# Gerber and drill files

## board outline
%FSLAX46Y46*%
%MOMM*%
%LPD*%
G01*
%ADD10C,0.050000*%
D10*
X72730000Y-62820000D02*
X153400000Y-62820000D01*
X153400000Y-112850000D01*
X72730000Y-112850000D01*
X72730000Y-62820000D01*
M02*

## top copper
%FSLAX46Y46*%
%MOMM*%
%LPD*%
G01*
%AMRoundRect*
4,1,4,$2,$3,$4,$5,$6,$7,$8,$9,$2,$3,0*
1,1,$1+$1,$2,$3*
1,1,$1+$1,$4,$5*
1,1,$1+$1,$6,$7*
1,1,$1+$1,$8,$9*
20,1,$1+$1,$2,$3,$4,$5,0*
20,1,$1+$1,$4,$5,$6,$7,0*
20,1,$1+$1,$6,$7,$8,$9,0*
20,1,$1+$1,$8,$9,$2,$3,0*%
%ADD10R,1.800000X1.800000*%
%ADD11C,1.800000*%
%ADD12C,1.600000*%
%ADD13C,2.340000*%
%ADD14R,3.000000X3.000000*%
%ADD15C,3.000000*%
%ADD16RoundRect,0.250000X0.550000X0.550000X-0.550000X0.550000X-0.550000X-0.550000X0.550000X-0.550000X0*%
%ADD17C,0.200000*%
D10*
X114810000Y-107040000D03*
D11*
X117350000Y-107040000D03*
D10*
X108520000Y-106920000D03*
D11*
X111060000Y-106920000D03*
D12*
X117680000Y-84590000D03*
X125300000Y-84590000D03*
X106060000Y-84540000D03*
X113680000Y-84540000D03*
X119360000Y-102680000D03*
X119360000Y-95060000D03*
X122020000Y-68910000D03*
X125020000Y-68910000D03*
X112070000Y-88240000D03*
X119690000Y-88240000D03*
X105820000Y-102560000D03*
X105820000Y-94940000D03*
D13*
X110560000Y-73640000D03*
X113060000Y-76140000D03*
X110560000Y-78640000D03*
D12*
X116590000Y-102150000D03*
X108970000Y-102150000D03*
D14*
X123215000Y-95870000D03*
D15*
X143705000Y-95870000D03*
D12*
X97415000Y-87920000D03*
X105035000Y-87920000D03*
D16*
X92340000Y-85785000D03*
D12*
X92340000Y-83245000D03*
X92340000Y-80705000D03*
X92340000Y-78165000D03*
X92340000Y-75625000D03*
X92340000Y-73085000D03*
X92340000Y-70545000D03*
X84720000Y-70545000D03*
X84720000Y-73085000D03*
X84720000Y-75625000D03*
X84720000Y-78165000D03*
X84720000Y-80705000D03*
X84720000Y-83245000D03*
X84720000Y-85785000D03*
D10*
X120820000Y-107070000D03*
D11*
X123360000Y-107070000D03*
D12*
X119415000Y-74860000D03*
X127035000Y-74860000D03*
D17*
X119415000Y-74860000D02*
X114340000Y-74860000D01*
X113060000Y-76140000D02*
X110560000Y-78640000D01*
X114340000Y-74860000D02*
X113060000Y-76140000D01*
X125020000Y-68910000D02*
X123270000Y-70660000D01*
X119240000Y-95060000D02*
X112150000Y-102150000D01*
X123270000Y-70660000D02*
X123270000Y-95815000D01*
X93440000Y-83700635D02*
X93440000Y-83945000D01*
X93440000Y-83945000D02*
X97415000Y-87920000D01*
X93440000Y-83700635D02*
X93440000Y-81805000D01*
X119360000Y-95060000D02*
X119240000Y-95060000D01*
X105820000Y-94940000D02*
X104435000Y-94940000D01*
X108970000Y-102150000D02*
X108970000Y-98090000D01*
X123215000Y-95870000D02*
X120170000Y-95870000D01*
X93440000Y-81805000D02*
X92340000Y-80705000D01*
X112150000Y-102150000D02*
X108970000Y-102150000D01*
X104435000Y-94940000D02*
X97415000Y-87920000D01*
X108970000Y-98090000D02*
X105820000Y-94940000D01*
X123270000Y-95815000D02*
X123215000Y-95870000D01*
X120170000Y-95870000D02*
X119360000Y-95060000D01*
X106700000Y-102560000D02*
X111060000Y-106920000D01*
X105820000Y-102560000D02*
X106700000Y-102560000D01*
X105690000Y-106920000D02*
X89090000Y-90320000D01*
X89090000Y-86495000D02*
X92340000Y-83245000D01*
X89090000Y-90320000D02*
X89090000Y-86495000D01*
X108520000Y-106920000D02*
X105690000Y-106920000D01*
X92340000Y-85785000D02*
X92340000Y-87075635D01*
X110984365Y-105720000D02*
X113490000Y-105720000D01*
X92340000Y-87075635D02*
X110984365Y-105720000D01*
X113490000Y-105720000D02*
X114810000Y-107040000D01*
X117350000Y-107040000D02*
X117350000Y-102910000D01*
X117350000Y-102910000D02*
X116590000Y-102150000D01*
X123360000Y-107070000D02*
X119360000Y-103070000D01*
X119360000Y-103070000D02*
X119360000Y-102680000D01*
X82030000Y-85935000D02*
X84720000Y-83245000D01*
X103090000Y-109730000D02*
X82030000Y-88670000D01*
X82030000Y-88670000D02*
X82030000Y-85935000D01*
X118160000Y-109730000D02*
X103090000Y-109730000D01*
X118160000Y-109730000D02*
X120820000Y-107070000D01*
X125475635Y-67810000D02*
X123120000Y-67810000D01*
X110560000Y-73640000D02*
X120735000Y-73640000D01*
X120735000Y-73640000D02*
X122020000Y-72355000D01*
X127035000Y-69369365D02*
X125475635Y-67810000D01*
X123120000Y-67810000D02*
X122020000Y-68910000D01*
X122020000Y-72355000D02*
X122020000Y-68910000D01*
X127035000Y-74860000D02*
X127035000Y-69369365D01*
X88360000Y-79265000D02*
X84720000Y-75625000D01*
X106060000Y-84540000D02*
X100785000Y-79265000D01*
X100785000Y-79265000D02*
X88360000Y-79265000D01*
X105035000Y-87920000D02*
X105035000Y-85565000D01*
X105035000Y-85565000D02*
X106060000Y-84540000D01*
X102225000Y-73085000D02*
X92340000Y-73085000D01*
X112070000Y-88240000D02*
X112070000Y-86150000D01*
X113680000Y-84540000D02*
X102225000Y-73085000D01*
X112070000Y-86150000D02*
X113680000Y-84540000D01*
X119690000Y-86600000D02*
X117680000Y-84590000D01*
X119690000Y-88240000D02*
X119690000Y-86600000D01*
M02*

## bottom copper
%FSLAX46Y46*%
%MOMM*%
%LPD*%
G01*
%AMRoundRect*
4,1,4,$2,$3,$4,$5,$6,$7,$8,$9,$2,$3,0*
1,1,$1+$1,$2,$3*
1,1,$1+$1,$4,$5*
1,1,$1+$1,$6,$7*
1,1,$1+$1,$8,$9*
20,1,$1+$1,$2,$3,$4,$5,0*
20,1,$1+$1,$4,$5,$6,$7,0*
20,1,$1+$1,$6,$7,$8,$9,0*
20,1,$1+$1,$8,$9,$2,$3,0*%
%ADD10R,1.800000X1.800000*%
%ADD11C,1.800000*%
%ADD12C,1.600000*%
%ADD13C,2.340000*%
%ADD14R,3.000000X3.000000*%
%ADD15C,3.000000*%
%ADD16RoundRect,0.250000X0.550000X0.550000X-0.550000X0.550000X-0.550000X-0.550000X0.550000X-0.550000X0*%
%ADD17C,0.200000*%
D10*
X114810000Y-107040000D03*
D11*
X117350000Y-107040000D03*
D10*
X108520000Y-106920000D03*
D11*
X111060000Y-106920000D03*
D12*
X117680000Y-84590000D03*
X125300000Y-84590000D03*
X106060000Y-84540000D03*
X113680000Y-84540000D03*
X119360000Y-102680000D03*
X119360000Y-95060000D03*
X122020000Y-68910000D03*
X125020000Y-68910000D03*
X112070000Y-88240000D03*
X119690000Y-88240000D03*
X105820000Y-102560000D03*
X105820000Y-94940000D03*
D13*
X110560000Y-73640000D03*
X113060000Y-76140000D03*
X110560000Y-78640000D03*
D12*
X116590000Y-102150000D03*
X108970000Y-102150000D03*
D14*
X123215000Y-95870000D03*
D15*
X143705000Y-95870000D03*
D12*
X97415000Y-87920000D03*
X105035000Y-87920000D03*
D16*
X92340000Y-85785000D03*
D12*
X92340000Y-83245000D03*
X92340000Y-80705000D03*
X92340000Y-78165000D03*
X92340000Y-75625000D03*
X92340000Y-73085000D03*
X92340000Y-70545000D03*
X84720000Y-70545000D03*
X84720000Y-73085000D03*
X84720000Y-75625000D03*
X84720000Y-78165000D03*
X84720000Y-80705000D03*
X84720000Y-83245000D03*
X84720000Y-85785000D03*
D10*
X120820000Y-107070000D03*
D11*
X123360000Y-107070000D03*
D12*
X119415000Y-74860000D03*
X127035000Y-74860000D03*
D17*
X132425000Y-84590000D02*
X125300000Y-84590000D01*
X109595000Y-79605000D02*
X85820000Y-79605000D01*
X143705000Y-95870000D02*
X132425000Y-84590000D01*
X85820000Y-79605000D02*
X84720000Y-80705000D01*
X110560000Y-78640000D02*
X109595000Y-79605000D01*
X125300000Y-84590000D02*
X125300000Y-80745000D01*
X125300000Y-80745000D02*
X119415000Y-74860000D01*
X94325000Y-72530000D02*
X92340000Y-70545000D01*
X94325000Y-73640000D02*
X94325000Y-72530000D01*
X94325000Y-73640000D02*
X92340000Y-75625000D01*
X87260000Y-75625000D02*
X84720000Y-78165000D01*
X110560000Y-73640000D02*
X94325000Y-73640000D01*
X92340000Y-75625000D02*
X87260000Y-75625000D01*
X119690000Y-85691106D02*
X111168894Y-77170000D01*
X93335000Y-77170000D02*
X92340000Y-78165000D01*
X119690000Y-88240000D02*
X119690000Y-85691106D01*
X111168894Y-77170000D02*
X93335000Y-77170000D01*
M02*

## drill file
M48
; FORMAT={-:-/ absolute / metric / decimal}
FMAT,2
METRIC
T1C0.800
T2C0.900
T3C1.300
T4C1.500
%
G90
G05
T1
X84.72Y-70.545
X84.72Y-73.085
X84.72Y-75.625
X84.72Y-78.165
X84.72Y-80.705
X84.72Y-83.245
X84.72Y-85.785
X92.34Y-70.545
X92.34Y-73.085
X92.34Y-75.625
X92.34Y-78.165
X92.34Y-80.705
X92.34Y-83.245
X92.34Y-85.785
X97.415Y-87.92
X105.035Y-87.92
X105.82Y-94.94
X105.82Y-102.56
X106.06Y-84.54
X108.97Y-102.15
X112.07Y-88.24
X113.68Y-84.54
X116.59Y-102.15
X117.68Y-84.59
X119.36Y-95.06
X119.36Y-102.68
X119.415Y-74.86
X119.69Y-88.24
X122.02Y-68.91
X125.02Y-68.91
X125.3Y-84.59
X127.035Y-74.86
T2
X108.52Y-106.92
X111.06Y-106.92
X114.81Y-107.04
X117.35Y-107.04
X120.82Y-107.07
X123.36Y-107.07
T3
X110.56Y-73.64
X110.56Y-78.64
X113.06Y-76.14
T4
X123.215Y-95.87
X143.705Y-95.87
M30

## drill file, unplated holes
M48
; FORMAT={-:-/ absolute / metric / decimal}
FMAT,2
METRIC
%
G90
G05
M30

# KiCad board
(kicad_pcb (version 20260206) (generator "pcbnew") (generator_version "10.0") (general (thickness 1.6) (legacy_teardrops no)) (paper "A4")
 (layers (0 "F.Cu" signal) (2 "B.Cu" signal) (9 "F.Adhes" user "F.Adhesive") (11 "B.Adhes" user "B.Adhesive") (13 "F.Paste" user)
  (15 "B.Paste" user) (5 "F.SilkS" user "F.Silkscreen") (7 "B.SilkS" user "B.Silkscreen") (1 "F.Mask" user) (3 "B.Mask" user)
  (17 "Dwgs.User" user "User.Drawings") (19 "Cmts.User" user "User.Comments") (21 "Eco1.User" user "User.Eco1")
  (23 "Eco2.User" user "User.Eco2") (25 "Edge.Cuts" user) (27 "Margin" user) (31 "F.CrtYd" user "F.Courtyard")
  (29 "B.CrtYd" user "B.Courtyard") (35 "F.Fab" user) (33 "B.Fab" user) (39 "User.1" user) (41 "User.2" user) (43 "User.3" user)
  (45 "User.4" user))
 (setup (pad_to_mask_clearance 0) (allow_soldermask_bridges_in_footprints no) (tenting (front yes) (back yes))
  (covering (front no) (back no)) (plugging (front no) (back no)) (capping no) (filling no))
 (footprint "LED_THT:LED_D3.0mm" (layer "F.Cu") (at 114.81 107.04)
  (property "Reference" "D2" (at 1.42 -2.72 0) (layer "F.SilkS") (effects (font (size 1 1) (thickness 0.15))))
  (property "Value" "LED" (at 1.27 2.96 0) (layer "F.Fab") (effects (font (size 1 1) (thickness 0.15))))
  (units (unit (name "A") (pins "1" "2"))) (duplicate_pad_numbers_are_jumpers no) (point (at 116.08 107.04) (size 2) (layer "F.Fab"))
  (pad "1" thru_hole rect (at 0 0) (size 1.8 1.8) (drill 0.9) (layers "*.Cu" "*.Mask") (remove_unused_layers no) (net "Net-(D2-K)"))
  (pad "2" thru_hole circle (at 2.54 0) (size 1.8 1.8) (drill 0.9) (layers "*.Cu" "*.Mask") (remove_unused_layers no) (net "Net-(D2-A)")))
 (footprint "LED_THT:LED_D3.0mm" (layer "F.Cu") (at 108.52 106.92)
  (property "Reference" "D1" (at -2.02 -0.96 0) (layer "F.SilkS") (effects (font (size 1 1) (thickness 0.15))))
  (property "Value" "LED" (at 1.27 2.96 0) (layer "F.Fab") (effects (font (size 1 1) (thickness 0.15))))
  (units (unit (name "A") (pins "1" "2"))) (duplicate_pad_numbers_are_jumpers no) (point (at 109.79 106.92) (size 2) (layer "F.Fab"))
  (pad "1" thru_hole rect (at 0 0) (size 1.8 1.8) (drill 0.9) (layers "*.Cu" "*.Mask") (remove_unused_layers no) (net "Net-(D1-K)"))
  (pad "2" thru_hole circle (at 2.54 0) (size 1.8 1.8) (drill 0.9) (layers "*.Cu" "*.Mask") (remove_unused_layers no) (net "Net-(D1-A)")))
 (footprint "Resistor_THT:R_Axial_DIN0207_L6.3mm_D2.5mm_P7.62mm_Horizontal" (layer "F.Cu") (at 117.68 84.59)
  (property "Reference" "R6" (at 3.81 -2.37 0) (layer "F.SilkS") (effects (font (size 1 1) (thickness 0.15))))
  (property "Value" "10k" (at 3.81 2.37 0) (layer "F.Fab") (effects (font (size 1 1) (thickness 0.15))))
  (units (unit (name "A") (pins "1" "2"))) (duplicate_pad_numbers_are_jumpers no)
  (pad "1" thru_hole circle (at 0 0) (size 1.6 1.6) (drill 0.8) (layers "*.Cu" "*.Mask") (remove_unused_layers no) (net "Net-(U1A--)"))
  (pad "2" thru_hole circle (at 7.62 0) (size 1.6 1.6) (drill 0.8) (layers "*.Cu" "*.Mask") (remove_unused_layers no) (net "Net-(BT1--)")))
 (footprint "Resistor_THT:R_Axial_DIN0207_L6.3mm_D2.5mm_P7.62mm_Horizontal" (layer "F.Cu") (at 106.06 84.54)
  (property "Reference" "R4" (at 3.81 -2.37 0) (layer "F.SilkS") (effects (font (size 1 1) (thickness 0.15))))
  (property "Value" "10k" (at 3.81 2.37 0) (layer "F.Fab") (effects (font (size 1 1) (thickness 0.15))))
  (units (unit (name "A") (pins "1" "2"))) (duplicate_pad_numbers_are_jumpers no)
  (pad "1" thru_hole circle (at 0 0) (size 1.6 1.6) (drill 0.8) (layers "*.Cu" "*.Mask") (remove_unused_layers no) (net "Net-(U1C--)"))
  (pad "2" thru_hole circle (at 7.62 0) (size 1.6 1.6) (drill 0.8) (layers "*.Cu" "*.Mask") (remove_unused_layers no) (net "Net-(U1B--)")))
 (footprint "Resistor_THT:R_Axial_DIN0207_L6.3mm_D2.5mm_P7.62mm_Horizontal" (layer "F.Cu") (at 119.36 102.68 90)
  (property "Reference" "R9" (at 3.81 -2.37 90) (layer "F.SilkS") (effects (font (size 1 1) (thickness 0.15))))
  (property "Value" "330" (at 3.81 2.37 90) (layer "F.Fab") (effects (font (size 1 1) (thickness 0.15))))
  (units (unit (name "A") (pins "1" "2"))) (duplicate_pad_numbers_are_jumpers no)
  (pad "1" thru_hole circle (at 0 0 90) (size 1.6 1.6) (drill 0.8) (layers "*.Cu" "*.Mask") (remove_unused_layers no) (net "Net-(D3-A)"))
  (pad "2" thru_hole circle (at 7.62 0 90) (size 1.6 1.6) (drill 0.8) (layers "*.Cu" "*.Mask") (remove_unused_layers no) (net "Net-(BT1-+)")))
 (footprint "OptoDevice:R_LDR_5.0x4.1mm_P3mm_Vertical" (layer "F.Cu") (at 122.02 68.91)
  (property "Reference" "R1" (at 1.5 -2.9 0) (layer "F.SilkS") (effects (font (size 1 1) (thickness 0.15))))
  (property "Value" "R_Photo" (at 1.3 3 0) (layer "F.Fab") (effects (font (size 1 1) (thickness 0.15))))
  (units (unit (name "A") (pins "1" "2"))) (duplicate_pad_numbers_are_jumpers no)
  (pad "1" thru_hole circle (at 0 0) (size 1.6 1.6) (drill 0.8) (layers "*.Cu" "*.Mask") (remove_unused_layers no) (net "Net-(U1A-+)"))
  (pad "2" thru_hole circle (at 3 0) (size 1.6 1.6) (drill 0.8) (layers "*.Cu" "*.Mask") (remove_unused_layers no) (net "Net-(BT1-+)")))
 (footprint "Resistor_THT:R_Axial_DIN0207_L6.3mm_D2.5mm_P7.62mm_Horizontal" (layer "F.Cu") (at 112.07 88.24)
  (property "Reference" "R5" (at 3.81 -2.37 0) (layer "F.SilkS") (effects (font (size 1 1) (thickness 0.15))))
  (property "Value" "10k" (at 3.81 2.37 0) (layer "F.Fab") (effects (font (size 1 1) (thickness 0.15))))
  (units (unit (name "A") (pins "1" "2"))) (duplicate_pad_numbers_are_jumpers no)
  (pad "1" thru_hole circle (at 0 0) (size 1.6 1.6) (drill 0.8) (layers "*.Cu" "*.Mask") (remove_unused_layers no) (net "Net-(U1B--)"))
  (pad "2" thru_hole circle (at 7.62 0) (size 1.6 1.6) (drill 0.8) (layers "*.Cu" "*.Mask") (remove_unused_layers no) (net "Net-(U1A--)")))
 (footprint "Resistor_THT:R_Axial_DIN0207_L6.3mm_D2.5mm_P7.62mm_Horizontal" (layer "F.Cu") (at 105.82 102.56 90)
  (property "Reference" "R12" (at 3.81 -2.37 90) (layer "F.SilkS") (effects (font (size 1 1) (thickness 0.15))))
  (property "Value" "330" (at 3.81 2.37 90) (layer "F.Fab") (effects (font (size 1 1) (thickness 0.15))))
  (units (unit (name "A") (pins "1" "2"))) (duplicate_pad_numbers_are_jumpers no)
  (pad "1" thru_hole circle (at 0 0 90) (size 1.6 1.6) (drill 0.8) (layers "*.Cu" "*.Mask") (remove_unused_layers no) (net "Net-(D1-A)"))
  (pad "2" thru_hole circle (at 7.62 0 90) (size 1.6 1.6) (drill 0.8) (layers "*.Cu" "*.Mask") (remove_unused_layers no) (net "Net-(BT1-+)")))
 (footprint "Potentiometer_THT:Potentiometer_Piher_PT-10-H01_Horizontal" (layer "F.Cu") (at 110.56 73.64)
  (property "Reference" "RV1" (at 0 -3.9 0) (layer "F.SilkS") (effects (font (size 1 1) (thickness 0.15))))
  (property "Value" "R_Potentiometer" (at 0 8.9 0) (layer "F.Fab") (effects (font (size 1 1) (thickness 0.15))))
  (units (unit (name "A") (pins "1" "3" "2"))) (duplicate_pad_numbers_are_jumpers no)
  (pad "1" thru_hole circle (at 0 0) (size 2.34 2.34) (drill 1.3) (layers "*.Cu" "*.Mask") (remove_unused_layers no) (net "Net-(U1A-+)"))
  (pad "2" thru_hole circle (at 2.5 2.5) (size 2.34 2.34) (drill 1.3) (layers "*.Cu" "*.Mask") (remove_unused_layers no) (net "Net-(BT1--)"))
  (pad "3" thru_hole circle (at 0 5) (size 2.34 2.34) (drill 1.3) (layers "*.Cu" "*.Mask") (remove_unused_layers no) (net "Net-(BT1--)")))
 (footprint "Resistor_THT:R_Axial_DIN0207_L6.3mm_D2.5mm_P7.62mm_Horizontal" (layer "F.Cu") (at 116.59 102.15 180)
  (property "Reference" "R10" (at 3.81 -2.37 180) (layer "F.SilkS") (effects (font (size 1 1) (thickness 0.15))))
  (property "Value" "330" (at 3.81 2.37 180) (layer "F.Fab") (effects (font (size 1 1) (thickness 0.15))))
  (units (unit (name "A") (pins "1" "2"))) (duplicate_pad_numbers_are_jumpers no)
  (pad "1" thru_hole circle (at 0 0 180) (size 1.6 1.6) (drill 0.8) (layers "*.Cu" "*.Mask") (remove_unused_layers no) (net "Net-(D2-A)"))
  (pad "2" thru_hole circle (at 7.62 0 180) (size 1.6 1.6) (drill 0.8) (layers "*.Cu" "*.Mask") (remove_unused_layers no)
   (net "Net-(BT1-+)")))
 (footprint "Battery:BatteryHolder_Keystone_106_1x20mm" (layer "F.Cu") (at 123.215 95.87)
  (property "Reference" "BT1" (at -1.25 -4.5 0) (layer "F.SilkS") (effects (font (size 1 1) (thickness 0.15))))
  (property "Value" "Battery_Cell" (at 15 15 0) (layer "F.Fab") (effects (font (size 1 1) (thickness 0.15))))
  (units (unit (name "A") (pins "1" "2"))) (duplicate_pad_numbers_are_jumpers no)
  (pad "1" thru_hole rect (at 0 0) (size 3 3) (drill 1.5) (layers "*.Cu" "*.Mask") (remove_unused_layers no) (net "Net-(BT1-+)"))
  (pad "2" thru_hole circle (at 20.49 0) (size 3 3) (drill 1.5) (layers "*.Cu" "*.Mask") (remove_unused_layers no) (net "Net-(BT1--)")))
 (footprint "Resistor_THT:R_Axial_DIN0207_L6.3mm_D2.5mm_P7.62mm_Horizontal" (layer "F.Cu") (at 97.415 87.92)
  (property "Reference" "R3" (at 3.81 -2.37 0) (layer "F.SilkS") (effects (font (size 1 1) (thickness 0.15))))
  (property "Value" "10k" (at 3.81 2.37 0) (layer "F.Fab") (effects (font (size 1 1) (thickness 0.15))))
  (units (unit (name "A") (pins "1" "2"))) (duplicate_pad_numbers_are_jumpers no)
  (pad "1" thru_hole circle (at 0 0) (size 1.6 1.6) (drill 0.8) (layers "*.Cu" "*.Mask") (remove_unused_layers no) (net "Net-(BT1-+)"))
  (pad "2" thru_hole circle (at 7.62 0) (size 1.6 1.6) (drill 0.8) (layers "*.Cu" "*.Mask") (remove_unused_layers no) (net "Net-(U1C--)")))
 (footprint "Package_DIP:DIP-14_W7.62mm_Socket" (layer "F.Cu") (at 92.34 85.785 180)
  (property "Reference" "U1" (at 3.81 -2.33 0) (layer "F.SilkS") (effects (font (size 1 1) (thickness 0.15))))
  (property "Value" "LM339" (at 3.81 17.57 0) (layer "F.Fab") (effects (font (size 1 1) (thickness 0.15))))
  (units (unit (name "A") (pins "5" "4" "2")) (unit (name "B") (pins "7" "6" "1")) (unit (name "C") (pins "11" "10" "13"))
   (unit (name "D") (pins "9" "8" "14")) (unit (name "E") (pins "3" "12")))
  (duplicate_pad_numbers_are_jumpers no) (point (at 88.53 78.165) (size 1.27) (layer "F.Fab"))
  (pad "1" thru_hole roundrect (at 0 0 180) (size 1.6 1.6) (drill 0.8) (layers "*.Cu" "*.Mask") (remove_unused_layers no)
   (roundrect_rratio 0.15625) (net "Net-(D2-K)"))
  (pad "2" thru_hole circle (at 0 2.54 180) (size 1.6 1.6) (drill 0.8) (layers "*.Cu" "*.Mask") (remove_unused_layers no) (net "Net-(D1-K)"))
  (pad "3" thru_hole circle (at 0 5.08 180) (size 1.6 1.6) (drill 0.8) (layers "*.Cu" "*.Mask") (remove_unused_layers no)
   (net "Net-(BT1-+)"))
  (pad "4" thru_hole circle (at 0 7.62 180) (size 1.6 1.6) (drill 0.8) (layers "*.Cu" "*.Mask") (remove_unused_layers no)
   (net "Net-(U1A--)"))
  (pad "5" thru_hole circle (at 0 10.16 180) (size 1.6 1.6) (drill 0.8) (layers "*.Cu" "*.Mask") (remove_unused_layers no)
   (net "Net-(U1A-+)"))
  (pad "6" thru_hole circle (at 0 12.7 180) (size 1.6 1.6) (drill 0.8) (layers "*.Cu" "*.Mask") (remove_unused_layers no)
   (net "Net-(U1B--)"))
  (pad "7" thru_hole circle (at 0 15.24 180) (size 1.6 1.6) (drill 0.8) (layers "*.Cu" "*.Mask") (remove_unused_layers no)
   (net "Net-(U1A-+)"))
  (pad "8" thru_hole circle (at 7.62 15.24 180) (size 1.6 1.6) (drill 0.8) (layers "*.Cu" "*.Mask") (remove_unused_layers no))
  (pad "9" thru_hole circle (at 7.62 12.7 180) (size 1.6 1.6) (drill 0.8) (layers "*.Cu" "*.Mask") (remove_unused_layers no))
  (pad "10" thru_hole circle (at 7.62 10.16 180) (size 1.6 1.6) (drill 0.8) (layers "*.Cu" "*.Mask") (remove_unused_layers no)
   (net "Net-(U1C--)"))
  (pad "11" thru_hole circle (at 7.62 7.62 180) (size 1.6 1.6) (drill 0.8) (layers "*.Cu" "*.Mask") (remove_unused_layers no)
   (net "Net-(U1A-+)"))
  (pad "12" thru_hole circle (at 7.62 5.08 180) (size 1.6 1.6) (drill 0.8) (layers "*.Cu" "*.Mask") (remove_unused_layers no)
   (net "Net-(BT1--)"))
  (pad "13" thru_hole circle (at 7.62 2.54 180) (size 1.6 1.6) (drill 0.8) (layers "*.Cu" "*.Mask") (remove_unused_layers no)
   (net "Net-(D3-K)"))
  (pad "14" thru_hole circle (at 7.62 0 180) (size 1.6 1.6) (drill 0.8) (layers "*.Cu" "*.Mask") (remove_unused_layers no)))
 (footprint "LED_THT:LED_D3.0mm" (layer "F.Cu") (at 120.82 107.07)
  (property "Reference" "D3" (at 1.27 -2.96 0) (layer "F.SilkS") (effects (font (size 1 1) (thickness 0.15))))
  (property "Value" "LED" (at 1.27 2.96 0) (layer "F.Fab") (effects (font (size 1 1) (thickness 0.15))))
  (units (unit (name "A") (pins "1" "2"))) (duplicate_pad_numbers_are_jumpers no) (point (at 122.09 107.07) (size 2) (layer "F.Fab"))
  (pad "1" thru_hole rect (at 0 0) (size 1.8 1.8) (drill 0.9) (layers "*.Cu" "*.Mask") (remove_unused_layers no) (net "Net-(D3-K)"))
  (pad "2" thru_hole circle (at 2.54 0) (size 1.8 1.8) (drill 0.9) (layers "*.Cu" "*.Mask") (remove_unused_layers no) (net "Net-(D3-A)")))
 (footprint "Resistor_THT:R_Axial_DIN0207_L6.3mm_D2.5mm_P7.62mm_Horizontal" (layer "F.Cu") (at 119.415 74.86)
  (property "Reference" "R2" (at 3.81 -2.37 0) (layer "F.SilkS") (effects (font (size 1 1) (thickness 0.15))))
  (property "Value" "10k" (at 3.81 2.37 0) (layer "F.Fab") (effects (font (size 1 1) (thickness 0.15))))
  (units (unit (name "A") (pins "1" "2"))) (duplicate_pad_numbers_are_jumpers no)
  (pad "1" thru_hole circle (at 0 0) (size 1.6 1.6) (drill 0.8) (layers "*.Cu" "*.Mask") (remove_unused_layers no) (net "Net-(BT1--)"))
  (pad "2" thru_hole circle (at 7.62 0) (size 1.6 1.6) (drill 0.8) (layers "*.Cu" "*.Mask") (remove_unused_layers no) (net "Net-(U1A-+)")))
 (gr_rect (start 72.73 62.82) (end 153.4 112.85) (stroke (width 0.05) (type default)) (fill no) (layer "Edge.Cuts"))
 (segment (start 119.415 74.86) (end 114.34 74.86) (width 0.2) (layer "F.Cu") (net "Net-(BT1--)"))
 (segment (start 113.06 76.14) (end 110.56 78.64) (width 0.2) (layer "F.Cu") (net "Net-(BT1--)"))
 (segment (start 114.34 74.86) (end 113.06 76.14) (width 0.2) (layer "F.Cu") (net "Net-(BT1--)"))
 (segment (start 132.425 84.59) (end 125.3 84.59) (width 0.2) (layer "B.Cu") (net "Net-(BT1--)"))
 (segment (start 109.595 79.605) (end 85.82 79.605) (width 0.2) (layer "B.Cu") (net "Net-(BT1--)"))
 (segment (start 143.705 95.87) (end 132.425 84.59) (width 0.2) (layer "B.Cu") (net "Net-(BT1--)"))
 (segment (start 85.82 79.605) (end 84.72 80.705) (width 0.2) (layer "B.Cu") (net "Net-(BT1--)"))
 (segment (start 110.56 78.64) (end 109.595 79.605) (width 0.2) (layer "B.Cu") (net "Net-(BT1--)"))
 (segment (start 125.3 84.59) (end 125.3 80.745) (width 0.2) (layer "B.Cu") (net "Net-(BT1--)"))
 (segment (start 125.3 80.745) (end 119.415 74.86) (width 0.2) (layer "B.Cu") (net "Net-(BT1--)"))
 (segment (start 125.02 68.91) (end 123.27 70.66) (width 0.2) (layer "F.Cu") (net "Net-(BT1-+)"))
 (segment (start 119.24 95.06) (end 112.15 102.15) (width 0.2) (layer "F.Cu") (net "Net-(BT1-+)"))
 (segment (start 123.27 70.66) (end 123.27 95.815) (width 0.2) (layer "F.Cu") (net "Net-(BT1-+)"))
 (segment (start 93.44 83.700635) (end 93.44 83.945) (width 0.2) (layer "F.Cu") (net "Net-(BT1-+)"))
 (segment (start 93.44 83.945) (end 97.415 87.92) (width 0.2) (layer "F.Cu") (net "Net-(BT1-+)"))
 (segment (start 93.44 83.700635) (end 93.44 81.805) (width 0.2) (layer "F.Cu") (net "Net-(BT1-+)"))
 (segment (start 119.36 95.06) (end 119.24 95.06) (width 0.2) (layer "F.Cu") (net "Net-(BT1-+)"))
 (segment (start 105.82 94.94) (end 104.435 94.94) (width 0.2) (layer "F.Cu") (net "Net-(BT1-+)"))
 (segment (start 108.97 102.15) (end 108.97 98.09) (width 0.2) (layer "F.Cu") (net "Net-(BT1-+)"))
 (segment (start 123.215 95.87) (end 120.17 95.87) (width 0.2) (layer "F.Cu") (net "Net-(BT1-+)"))
 (segment (start 93.44 81.805) (end 92.34 80.705) (width 0.2) (layer "F.Cu") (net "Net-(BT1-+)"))
 (segment (start 112.15 102.15) (end 108.97 102.15) (width 0.2) (layer "F.Cu") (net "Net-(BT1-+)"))
 (segment (start 104.435 94.94) (end 97.415 87.92) (width 0.2) (layer "F.Cu") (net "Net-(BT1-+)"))
 (segment (start 108.97 98.09) (end 105.82 94.94) (width 0.2) (layer "F.Cu") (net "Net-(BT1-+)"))
 (segment (start 123.27 95.815) (end 123.215 95.87) (width 0.2) (layer "F.Cu") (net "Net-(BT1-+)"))
 (segment (start 120.17 95.87) (end 119.36 95.06) (width 0.2) (layer "F.Cu") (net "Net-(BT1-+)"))
 (segment (start 106.7 102.56) (end 111.06 106.92) (width 0.2) (layer "F.Cu") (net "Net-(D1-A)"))
 (segment (start 105.82 102.56) (end 106.7 102.56) (width 0.2) (layer "F.Cu") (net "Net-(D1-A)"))
 (segment (start 105.69 106.92) (end 89.09 90.32) (width 0.2) (layer "F.Cu") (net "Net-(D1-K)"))
 (segment (start 89.09 86.495) (end 92.34 83.245) (width 0.2) (layer "F.Cu") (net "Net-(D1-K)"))
 (segment (start 89.09 90.32) (end 89.09 86.495) (width 0.2) (layer "F.Cu") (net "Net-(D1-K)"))
 (segment (start 108.52 106.92) (end 105.69 106.92) (width 0.2) (layer "F.Cu") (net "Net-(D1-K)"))
 (segment (start 92.34 85.785) (end 92.34 87.075635) (width 0.2) (layer "F.Cu") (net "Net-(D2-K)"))
 (segment (start 110.984365 105.72) (end 113.49 105.72) (width 0.2) (layer "F.Cu") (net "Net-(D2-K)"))
 (segment (start 92.34 87.075635) (end 110.984365 105.72) (width 0.2) (layer "F.Cu") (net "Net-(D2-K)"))
 (segment (start 113.49 105.72) (end 114.81 107.04) (width 0.2) (layer "F.Cu") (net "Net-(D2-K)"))
 (segment (start 117.35 107.04) (end 117.35 102.91) (width 0.2) (layer "F.Cu") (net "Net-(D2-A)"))
 (segment (start 117.35 102.91) (end 116.59 102.15) (width 0.2) (layer "F.Cu") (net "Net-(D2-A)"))
 (segment (start 123.36 107.07) (end 119.36 103.07) (width 0.2) (layer "F.Cu") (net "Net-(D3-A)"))
 (segment (start 119.36 103.07) (end 119.36 102.68) (width 0.2) (layer "F.Cu") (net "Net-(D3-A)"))
 (segment (start 82.03 85.935) (end 84.72 83.245) (width 0.2) (layer "F.Cu") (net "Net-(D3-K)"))
 (segment (start 103.09 109.73) (end 82.03 88.67) (width 0.2) (layer "F.Cu") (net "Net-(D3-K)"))
 (segment (start 82.03 88.67) (end 82.03 85.935) (width 0.2) (layer "F.Cu") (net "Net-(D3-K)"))
 (segment (start 118.16 109.73) (end 103.09 109.73) (width 0.2) (layer "F.Cu") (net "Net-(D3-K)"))
 (segment (start 118.16 109.73) (end 120.82 107.07) (width 0.2) (layer "F.Cu") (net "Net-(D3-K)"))
 (segment (start 125.475635 67.81) (end 123.12 67.81) (width 0.2) (layer "F.Cu") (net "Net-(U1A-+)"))
 (segment (start 110.56 73.64) (end 120.735 73.64) (width 0.2) (layer "F.Cu") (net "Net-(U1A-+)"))
 (segment (start 120.735 73.64) (end 122.02 72.355) (width 0.2) (layer "F.Cu") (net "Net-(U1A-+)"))
 (segment (start 127.035 69.369365) (end 125.475635 67.81) (width 0.2) (layer "F.Cu") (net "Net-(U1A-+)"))
 (segment (start 123.12 67.81) (end 122.02 68.91) (width 0.2) (layer "F.Cu") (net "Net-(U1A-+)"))
 (segment (start 122.02 72.355) (end 122.02 68.91) (width 0.2) (layer "F.Cu") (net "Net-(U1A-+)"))
 (segment (start 127.035 74.86) (end 127.035 69.369365) (width 0.2) (layer "F.Cu") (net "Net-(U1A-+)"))
 (segment (start 94.325 72.53) (end 92.34 70.545) (width 0.2) (layer "B.Cu") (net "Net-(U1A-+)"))
 (segment (start 94.325 73.64) (end 94.325 72.53) (width 0.2) (layer "B.Cu") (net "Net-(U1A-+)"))
 (segment (start 94.325 73.64) (end 92.34 75.625) (width 0.2) (layer "B.Cu") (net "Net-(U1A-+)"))
 (segment (start 87.26 75.625) (end 84.72 78.165) (width 0.2) (layer "B.Cu") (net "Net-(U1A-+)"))
 (segment (start 110.56 73.64) (end 94.325 73.64) (width 0.2) (layer "B.Cu") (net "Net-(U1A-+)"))
 (segment (start 92.34 75.625) (end 87.26 75.625) (width 0.2) (layer "B.Cu") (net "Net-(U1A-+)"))
 (segment (start 88.36 79.265) (end 84.72 75.625) (width 0.2) (layer "F.Cu") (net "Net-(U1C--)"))
 (segment (start 106.06 84.54) (end 100.785 79.265) (width 0.2) (layer "F.Cu") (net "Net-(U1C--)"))
 (segment (start 100.785 79.265) (end 88.36 79.265) (width 0.2) (layer "F.Cu") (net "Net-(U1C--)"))
 (segment (start 105.035 87.92) (end 105.035 85.565) (width 0.2) (layer "F.Cu") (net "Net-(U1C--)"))
 (segment (start 105.035 85.565) (end 106.06 84.54) (width 0.2) (layer "F.Cu") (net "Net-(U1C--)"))
 (segment (start 102.225 73.085) (end 92.34 73.085) (width 0.2) (layer "F.Cu") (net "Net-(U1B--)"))
 (segment (start 112.07 88.24) (end 112.07 86.15) (width 0.2) (layer "F.Cu") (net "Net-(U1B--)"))
 (segment (start 113.68 84.54) (end 102.225 73.085) (width 0.2) (layer "F.Cu") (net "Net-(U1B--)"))
 (segment (start 112.07 86.15) (end 113.68 84.54) (width 0.2) (layer "F.Cu") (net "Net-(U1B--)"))
 (segment (start 119.69 86.6) (end 117.68 84.59) (width 0.2) (layer "F.Cu") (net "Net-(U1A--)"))
 (segment (start 119.69 88.24) (end 119.69 86.6) (width 0.2) (layer "F.Cu") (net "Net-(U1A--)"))
 (segment (start 119.69 85.691106) (end 111.168894 77.17) (width 0.2) (layer "B.Cu") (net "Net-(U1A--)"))
 (segment (start 93.335 77.17) (end 92.34 78.165) (width 0.2) (layer "B.Cu") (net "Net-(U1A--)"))
 (segment (start 119.69 88.24) (end 119.69 85.691106) (width 0.2) (layer "B.Cu") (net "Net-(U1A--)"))
 (segment (start 111.168894 77.17) (end 93.335 77.17) (width 0.2) (layer "B.Cu") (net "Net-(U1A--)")))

